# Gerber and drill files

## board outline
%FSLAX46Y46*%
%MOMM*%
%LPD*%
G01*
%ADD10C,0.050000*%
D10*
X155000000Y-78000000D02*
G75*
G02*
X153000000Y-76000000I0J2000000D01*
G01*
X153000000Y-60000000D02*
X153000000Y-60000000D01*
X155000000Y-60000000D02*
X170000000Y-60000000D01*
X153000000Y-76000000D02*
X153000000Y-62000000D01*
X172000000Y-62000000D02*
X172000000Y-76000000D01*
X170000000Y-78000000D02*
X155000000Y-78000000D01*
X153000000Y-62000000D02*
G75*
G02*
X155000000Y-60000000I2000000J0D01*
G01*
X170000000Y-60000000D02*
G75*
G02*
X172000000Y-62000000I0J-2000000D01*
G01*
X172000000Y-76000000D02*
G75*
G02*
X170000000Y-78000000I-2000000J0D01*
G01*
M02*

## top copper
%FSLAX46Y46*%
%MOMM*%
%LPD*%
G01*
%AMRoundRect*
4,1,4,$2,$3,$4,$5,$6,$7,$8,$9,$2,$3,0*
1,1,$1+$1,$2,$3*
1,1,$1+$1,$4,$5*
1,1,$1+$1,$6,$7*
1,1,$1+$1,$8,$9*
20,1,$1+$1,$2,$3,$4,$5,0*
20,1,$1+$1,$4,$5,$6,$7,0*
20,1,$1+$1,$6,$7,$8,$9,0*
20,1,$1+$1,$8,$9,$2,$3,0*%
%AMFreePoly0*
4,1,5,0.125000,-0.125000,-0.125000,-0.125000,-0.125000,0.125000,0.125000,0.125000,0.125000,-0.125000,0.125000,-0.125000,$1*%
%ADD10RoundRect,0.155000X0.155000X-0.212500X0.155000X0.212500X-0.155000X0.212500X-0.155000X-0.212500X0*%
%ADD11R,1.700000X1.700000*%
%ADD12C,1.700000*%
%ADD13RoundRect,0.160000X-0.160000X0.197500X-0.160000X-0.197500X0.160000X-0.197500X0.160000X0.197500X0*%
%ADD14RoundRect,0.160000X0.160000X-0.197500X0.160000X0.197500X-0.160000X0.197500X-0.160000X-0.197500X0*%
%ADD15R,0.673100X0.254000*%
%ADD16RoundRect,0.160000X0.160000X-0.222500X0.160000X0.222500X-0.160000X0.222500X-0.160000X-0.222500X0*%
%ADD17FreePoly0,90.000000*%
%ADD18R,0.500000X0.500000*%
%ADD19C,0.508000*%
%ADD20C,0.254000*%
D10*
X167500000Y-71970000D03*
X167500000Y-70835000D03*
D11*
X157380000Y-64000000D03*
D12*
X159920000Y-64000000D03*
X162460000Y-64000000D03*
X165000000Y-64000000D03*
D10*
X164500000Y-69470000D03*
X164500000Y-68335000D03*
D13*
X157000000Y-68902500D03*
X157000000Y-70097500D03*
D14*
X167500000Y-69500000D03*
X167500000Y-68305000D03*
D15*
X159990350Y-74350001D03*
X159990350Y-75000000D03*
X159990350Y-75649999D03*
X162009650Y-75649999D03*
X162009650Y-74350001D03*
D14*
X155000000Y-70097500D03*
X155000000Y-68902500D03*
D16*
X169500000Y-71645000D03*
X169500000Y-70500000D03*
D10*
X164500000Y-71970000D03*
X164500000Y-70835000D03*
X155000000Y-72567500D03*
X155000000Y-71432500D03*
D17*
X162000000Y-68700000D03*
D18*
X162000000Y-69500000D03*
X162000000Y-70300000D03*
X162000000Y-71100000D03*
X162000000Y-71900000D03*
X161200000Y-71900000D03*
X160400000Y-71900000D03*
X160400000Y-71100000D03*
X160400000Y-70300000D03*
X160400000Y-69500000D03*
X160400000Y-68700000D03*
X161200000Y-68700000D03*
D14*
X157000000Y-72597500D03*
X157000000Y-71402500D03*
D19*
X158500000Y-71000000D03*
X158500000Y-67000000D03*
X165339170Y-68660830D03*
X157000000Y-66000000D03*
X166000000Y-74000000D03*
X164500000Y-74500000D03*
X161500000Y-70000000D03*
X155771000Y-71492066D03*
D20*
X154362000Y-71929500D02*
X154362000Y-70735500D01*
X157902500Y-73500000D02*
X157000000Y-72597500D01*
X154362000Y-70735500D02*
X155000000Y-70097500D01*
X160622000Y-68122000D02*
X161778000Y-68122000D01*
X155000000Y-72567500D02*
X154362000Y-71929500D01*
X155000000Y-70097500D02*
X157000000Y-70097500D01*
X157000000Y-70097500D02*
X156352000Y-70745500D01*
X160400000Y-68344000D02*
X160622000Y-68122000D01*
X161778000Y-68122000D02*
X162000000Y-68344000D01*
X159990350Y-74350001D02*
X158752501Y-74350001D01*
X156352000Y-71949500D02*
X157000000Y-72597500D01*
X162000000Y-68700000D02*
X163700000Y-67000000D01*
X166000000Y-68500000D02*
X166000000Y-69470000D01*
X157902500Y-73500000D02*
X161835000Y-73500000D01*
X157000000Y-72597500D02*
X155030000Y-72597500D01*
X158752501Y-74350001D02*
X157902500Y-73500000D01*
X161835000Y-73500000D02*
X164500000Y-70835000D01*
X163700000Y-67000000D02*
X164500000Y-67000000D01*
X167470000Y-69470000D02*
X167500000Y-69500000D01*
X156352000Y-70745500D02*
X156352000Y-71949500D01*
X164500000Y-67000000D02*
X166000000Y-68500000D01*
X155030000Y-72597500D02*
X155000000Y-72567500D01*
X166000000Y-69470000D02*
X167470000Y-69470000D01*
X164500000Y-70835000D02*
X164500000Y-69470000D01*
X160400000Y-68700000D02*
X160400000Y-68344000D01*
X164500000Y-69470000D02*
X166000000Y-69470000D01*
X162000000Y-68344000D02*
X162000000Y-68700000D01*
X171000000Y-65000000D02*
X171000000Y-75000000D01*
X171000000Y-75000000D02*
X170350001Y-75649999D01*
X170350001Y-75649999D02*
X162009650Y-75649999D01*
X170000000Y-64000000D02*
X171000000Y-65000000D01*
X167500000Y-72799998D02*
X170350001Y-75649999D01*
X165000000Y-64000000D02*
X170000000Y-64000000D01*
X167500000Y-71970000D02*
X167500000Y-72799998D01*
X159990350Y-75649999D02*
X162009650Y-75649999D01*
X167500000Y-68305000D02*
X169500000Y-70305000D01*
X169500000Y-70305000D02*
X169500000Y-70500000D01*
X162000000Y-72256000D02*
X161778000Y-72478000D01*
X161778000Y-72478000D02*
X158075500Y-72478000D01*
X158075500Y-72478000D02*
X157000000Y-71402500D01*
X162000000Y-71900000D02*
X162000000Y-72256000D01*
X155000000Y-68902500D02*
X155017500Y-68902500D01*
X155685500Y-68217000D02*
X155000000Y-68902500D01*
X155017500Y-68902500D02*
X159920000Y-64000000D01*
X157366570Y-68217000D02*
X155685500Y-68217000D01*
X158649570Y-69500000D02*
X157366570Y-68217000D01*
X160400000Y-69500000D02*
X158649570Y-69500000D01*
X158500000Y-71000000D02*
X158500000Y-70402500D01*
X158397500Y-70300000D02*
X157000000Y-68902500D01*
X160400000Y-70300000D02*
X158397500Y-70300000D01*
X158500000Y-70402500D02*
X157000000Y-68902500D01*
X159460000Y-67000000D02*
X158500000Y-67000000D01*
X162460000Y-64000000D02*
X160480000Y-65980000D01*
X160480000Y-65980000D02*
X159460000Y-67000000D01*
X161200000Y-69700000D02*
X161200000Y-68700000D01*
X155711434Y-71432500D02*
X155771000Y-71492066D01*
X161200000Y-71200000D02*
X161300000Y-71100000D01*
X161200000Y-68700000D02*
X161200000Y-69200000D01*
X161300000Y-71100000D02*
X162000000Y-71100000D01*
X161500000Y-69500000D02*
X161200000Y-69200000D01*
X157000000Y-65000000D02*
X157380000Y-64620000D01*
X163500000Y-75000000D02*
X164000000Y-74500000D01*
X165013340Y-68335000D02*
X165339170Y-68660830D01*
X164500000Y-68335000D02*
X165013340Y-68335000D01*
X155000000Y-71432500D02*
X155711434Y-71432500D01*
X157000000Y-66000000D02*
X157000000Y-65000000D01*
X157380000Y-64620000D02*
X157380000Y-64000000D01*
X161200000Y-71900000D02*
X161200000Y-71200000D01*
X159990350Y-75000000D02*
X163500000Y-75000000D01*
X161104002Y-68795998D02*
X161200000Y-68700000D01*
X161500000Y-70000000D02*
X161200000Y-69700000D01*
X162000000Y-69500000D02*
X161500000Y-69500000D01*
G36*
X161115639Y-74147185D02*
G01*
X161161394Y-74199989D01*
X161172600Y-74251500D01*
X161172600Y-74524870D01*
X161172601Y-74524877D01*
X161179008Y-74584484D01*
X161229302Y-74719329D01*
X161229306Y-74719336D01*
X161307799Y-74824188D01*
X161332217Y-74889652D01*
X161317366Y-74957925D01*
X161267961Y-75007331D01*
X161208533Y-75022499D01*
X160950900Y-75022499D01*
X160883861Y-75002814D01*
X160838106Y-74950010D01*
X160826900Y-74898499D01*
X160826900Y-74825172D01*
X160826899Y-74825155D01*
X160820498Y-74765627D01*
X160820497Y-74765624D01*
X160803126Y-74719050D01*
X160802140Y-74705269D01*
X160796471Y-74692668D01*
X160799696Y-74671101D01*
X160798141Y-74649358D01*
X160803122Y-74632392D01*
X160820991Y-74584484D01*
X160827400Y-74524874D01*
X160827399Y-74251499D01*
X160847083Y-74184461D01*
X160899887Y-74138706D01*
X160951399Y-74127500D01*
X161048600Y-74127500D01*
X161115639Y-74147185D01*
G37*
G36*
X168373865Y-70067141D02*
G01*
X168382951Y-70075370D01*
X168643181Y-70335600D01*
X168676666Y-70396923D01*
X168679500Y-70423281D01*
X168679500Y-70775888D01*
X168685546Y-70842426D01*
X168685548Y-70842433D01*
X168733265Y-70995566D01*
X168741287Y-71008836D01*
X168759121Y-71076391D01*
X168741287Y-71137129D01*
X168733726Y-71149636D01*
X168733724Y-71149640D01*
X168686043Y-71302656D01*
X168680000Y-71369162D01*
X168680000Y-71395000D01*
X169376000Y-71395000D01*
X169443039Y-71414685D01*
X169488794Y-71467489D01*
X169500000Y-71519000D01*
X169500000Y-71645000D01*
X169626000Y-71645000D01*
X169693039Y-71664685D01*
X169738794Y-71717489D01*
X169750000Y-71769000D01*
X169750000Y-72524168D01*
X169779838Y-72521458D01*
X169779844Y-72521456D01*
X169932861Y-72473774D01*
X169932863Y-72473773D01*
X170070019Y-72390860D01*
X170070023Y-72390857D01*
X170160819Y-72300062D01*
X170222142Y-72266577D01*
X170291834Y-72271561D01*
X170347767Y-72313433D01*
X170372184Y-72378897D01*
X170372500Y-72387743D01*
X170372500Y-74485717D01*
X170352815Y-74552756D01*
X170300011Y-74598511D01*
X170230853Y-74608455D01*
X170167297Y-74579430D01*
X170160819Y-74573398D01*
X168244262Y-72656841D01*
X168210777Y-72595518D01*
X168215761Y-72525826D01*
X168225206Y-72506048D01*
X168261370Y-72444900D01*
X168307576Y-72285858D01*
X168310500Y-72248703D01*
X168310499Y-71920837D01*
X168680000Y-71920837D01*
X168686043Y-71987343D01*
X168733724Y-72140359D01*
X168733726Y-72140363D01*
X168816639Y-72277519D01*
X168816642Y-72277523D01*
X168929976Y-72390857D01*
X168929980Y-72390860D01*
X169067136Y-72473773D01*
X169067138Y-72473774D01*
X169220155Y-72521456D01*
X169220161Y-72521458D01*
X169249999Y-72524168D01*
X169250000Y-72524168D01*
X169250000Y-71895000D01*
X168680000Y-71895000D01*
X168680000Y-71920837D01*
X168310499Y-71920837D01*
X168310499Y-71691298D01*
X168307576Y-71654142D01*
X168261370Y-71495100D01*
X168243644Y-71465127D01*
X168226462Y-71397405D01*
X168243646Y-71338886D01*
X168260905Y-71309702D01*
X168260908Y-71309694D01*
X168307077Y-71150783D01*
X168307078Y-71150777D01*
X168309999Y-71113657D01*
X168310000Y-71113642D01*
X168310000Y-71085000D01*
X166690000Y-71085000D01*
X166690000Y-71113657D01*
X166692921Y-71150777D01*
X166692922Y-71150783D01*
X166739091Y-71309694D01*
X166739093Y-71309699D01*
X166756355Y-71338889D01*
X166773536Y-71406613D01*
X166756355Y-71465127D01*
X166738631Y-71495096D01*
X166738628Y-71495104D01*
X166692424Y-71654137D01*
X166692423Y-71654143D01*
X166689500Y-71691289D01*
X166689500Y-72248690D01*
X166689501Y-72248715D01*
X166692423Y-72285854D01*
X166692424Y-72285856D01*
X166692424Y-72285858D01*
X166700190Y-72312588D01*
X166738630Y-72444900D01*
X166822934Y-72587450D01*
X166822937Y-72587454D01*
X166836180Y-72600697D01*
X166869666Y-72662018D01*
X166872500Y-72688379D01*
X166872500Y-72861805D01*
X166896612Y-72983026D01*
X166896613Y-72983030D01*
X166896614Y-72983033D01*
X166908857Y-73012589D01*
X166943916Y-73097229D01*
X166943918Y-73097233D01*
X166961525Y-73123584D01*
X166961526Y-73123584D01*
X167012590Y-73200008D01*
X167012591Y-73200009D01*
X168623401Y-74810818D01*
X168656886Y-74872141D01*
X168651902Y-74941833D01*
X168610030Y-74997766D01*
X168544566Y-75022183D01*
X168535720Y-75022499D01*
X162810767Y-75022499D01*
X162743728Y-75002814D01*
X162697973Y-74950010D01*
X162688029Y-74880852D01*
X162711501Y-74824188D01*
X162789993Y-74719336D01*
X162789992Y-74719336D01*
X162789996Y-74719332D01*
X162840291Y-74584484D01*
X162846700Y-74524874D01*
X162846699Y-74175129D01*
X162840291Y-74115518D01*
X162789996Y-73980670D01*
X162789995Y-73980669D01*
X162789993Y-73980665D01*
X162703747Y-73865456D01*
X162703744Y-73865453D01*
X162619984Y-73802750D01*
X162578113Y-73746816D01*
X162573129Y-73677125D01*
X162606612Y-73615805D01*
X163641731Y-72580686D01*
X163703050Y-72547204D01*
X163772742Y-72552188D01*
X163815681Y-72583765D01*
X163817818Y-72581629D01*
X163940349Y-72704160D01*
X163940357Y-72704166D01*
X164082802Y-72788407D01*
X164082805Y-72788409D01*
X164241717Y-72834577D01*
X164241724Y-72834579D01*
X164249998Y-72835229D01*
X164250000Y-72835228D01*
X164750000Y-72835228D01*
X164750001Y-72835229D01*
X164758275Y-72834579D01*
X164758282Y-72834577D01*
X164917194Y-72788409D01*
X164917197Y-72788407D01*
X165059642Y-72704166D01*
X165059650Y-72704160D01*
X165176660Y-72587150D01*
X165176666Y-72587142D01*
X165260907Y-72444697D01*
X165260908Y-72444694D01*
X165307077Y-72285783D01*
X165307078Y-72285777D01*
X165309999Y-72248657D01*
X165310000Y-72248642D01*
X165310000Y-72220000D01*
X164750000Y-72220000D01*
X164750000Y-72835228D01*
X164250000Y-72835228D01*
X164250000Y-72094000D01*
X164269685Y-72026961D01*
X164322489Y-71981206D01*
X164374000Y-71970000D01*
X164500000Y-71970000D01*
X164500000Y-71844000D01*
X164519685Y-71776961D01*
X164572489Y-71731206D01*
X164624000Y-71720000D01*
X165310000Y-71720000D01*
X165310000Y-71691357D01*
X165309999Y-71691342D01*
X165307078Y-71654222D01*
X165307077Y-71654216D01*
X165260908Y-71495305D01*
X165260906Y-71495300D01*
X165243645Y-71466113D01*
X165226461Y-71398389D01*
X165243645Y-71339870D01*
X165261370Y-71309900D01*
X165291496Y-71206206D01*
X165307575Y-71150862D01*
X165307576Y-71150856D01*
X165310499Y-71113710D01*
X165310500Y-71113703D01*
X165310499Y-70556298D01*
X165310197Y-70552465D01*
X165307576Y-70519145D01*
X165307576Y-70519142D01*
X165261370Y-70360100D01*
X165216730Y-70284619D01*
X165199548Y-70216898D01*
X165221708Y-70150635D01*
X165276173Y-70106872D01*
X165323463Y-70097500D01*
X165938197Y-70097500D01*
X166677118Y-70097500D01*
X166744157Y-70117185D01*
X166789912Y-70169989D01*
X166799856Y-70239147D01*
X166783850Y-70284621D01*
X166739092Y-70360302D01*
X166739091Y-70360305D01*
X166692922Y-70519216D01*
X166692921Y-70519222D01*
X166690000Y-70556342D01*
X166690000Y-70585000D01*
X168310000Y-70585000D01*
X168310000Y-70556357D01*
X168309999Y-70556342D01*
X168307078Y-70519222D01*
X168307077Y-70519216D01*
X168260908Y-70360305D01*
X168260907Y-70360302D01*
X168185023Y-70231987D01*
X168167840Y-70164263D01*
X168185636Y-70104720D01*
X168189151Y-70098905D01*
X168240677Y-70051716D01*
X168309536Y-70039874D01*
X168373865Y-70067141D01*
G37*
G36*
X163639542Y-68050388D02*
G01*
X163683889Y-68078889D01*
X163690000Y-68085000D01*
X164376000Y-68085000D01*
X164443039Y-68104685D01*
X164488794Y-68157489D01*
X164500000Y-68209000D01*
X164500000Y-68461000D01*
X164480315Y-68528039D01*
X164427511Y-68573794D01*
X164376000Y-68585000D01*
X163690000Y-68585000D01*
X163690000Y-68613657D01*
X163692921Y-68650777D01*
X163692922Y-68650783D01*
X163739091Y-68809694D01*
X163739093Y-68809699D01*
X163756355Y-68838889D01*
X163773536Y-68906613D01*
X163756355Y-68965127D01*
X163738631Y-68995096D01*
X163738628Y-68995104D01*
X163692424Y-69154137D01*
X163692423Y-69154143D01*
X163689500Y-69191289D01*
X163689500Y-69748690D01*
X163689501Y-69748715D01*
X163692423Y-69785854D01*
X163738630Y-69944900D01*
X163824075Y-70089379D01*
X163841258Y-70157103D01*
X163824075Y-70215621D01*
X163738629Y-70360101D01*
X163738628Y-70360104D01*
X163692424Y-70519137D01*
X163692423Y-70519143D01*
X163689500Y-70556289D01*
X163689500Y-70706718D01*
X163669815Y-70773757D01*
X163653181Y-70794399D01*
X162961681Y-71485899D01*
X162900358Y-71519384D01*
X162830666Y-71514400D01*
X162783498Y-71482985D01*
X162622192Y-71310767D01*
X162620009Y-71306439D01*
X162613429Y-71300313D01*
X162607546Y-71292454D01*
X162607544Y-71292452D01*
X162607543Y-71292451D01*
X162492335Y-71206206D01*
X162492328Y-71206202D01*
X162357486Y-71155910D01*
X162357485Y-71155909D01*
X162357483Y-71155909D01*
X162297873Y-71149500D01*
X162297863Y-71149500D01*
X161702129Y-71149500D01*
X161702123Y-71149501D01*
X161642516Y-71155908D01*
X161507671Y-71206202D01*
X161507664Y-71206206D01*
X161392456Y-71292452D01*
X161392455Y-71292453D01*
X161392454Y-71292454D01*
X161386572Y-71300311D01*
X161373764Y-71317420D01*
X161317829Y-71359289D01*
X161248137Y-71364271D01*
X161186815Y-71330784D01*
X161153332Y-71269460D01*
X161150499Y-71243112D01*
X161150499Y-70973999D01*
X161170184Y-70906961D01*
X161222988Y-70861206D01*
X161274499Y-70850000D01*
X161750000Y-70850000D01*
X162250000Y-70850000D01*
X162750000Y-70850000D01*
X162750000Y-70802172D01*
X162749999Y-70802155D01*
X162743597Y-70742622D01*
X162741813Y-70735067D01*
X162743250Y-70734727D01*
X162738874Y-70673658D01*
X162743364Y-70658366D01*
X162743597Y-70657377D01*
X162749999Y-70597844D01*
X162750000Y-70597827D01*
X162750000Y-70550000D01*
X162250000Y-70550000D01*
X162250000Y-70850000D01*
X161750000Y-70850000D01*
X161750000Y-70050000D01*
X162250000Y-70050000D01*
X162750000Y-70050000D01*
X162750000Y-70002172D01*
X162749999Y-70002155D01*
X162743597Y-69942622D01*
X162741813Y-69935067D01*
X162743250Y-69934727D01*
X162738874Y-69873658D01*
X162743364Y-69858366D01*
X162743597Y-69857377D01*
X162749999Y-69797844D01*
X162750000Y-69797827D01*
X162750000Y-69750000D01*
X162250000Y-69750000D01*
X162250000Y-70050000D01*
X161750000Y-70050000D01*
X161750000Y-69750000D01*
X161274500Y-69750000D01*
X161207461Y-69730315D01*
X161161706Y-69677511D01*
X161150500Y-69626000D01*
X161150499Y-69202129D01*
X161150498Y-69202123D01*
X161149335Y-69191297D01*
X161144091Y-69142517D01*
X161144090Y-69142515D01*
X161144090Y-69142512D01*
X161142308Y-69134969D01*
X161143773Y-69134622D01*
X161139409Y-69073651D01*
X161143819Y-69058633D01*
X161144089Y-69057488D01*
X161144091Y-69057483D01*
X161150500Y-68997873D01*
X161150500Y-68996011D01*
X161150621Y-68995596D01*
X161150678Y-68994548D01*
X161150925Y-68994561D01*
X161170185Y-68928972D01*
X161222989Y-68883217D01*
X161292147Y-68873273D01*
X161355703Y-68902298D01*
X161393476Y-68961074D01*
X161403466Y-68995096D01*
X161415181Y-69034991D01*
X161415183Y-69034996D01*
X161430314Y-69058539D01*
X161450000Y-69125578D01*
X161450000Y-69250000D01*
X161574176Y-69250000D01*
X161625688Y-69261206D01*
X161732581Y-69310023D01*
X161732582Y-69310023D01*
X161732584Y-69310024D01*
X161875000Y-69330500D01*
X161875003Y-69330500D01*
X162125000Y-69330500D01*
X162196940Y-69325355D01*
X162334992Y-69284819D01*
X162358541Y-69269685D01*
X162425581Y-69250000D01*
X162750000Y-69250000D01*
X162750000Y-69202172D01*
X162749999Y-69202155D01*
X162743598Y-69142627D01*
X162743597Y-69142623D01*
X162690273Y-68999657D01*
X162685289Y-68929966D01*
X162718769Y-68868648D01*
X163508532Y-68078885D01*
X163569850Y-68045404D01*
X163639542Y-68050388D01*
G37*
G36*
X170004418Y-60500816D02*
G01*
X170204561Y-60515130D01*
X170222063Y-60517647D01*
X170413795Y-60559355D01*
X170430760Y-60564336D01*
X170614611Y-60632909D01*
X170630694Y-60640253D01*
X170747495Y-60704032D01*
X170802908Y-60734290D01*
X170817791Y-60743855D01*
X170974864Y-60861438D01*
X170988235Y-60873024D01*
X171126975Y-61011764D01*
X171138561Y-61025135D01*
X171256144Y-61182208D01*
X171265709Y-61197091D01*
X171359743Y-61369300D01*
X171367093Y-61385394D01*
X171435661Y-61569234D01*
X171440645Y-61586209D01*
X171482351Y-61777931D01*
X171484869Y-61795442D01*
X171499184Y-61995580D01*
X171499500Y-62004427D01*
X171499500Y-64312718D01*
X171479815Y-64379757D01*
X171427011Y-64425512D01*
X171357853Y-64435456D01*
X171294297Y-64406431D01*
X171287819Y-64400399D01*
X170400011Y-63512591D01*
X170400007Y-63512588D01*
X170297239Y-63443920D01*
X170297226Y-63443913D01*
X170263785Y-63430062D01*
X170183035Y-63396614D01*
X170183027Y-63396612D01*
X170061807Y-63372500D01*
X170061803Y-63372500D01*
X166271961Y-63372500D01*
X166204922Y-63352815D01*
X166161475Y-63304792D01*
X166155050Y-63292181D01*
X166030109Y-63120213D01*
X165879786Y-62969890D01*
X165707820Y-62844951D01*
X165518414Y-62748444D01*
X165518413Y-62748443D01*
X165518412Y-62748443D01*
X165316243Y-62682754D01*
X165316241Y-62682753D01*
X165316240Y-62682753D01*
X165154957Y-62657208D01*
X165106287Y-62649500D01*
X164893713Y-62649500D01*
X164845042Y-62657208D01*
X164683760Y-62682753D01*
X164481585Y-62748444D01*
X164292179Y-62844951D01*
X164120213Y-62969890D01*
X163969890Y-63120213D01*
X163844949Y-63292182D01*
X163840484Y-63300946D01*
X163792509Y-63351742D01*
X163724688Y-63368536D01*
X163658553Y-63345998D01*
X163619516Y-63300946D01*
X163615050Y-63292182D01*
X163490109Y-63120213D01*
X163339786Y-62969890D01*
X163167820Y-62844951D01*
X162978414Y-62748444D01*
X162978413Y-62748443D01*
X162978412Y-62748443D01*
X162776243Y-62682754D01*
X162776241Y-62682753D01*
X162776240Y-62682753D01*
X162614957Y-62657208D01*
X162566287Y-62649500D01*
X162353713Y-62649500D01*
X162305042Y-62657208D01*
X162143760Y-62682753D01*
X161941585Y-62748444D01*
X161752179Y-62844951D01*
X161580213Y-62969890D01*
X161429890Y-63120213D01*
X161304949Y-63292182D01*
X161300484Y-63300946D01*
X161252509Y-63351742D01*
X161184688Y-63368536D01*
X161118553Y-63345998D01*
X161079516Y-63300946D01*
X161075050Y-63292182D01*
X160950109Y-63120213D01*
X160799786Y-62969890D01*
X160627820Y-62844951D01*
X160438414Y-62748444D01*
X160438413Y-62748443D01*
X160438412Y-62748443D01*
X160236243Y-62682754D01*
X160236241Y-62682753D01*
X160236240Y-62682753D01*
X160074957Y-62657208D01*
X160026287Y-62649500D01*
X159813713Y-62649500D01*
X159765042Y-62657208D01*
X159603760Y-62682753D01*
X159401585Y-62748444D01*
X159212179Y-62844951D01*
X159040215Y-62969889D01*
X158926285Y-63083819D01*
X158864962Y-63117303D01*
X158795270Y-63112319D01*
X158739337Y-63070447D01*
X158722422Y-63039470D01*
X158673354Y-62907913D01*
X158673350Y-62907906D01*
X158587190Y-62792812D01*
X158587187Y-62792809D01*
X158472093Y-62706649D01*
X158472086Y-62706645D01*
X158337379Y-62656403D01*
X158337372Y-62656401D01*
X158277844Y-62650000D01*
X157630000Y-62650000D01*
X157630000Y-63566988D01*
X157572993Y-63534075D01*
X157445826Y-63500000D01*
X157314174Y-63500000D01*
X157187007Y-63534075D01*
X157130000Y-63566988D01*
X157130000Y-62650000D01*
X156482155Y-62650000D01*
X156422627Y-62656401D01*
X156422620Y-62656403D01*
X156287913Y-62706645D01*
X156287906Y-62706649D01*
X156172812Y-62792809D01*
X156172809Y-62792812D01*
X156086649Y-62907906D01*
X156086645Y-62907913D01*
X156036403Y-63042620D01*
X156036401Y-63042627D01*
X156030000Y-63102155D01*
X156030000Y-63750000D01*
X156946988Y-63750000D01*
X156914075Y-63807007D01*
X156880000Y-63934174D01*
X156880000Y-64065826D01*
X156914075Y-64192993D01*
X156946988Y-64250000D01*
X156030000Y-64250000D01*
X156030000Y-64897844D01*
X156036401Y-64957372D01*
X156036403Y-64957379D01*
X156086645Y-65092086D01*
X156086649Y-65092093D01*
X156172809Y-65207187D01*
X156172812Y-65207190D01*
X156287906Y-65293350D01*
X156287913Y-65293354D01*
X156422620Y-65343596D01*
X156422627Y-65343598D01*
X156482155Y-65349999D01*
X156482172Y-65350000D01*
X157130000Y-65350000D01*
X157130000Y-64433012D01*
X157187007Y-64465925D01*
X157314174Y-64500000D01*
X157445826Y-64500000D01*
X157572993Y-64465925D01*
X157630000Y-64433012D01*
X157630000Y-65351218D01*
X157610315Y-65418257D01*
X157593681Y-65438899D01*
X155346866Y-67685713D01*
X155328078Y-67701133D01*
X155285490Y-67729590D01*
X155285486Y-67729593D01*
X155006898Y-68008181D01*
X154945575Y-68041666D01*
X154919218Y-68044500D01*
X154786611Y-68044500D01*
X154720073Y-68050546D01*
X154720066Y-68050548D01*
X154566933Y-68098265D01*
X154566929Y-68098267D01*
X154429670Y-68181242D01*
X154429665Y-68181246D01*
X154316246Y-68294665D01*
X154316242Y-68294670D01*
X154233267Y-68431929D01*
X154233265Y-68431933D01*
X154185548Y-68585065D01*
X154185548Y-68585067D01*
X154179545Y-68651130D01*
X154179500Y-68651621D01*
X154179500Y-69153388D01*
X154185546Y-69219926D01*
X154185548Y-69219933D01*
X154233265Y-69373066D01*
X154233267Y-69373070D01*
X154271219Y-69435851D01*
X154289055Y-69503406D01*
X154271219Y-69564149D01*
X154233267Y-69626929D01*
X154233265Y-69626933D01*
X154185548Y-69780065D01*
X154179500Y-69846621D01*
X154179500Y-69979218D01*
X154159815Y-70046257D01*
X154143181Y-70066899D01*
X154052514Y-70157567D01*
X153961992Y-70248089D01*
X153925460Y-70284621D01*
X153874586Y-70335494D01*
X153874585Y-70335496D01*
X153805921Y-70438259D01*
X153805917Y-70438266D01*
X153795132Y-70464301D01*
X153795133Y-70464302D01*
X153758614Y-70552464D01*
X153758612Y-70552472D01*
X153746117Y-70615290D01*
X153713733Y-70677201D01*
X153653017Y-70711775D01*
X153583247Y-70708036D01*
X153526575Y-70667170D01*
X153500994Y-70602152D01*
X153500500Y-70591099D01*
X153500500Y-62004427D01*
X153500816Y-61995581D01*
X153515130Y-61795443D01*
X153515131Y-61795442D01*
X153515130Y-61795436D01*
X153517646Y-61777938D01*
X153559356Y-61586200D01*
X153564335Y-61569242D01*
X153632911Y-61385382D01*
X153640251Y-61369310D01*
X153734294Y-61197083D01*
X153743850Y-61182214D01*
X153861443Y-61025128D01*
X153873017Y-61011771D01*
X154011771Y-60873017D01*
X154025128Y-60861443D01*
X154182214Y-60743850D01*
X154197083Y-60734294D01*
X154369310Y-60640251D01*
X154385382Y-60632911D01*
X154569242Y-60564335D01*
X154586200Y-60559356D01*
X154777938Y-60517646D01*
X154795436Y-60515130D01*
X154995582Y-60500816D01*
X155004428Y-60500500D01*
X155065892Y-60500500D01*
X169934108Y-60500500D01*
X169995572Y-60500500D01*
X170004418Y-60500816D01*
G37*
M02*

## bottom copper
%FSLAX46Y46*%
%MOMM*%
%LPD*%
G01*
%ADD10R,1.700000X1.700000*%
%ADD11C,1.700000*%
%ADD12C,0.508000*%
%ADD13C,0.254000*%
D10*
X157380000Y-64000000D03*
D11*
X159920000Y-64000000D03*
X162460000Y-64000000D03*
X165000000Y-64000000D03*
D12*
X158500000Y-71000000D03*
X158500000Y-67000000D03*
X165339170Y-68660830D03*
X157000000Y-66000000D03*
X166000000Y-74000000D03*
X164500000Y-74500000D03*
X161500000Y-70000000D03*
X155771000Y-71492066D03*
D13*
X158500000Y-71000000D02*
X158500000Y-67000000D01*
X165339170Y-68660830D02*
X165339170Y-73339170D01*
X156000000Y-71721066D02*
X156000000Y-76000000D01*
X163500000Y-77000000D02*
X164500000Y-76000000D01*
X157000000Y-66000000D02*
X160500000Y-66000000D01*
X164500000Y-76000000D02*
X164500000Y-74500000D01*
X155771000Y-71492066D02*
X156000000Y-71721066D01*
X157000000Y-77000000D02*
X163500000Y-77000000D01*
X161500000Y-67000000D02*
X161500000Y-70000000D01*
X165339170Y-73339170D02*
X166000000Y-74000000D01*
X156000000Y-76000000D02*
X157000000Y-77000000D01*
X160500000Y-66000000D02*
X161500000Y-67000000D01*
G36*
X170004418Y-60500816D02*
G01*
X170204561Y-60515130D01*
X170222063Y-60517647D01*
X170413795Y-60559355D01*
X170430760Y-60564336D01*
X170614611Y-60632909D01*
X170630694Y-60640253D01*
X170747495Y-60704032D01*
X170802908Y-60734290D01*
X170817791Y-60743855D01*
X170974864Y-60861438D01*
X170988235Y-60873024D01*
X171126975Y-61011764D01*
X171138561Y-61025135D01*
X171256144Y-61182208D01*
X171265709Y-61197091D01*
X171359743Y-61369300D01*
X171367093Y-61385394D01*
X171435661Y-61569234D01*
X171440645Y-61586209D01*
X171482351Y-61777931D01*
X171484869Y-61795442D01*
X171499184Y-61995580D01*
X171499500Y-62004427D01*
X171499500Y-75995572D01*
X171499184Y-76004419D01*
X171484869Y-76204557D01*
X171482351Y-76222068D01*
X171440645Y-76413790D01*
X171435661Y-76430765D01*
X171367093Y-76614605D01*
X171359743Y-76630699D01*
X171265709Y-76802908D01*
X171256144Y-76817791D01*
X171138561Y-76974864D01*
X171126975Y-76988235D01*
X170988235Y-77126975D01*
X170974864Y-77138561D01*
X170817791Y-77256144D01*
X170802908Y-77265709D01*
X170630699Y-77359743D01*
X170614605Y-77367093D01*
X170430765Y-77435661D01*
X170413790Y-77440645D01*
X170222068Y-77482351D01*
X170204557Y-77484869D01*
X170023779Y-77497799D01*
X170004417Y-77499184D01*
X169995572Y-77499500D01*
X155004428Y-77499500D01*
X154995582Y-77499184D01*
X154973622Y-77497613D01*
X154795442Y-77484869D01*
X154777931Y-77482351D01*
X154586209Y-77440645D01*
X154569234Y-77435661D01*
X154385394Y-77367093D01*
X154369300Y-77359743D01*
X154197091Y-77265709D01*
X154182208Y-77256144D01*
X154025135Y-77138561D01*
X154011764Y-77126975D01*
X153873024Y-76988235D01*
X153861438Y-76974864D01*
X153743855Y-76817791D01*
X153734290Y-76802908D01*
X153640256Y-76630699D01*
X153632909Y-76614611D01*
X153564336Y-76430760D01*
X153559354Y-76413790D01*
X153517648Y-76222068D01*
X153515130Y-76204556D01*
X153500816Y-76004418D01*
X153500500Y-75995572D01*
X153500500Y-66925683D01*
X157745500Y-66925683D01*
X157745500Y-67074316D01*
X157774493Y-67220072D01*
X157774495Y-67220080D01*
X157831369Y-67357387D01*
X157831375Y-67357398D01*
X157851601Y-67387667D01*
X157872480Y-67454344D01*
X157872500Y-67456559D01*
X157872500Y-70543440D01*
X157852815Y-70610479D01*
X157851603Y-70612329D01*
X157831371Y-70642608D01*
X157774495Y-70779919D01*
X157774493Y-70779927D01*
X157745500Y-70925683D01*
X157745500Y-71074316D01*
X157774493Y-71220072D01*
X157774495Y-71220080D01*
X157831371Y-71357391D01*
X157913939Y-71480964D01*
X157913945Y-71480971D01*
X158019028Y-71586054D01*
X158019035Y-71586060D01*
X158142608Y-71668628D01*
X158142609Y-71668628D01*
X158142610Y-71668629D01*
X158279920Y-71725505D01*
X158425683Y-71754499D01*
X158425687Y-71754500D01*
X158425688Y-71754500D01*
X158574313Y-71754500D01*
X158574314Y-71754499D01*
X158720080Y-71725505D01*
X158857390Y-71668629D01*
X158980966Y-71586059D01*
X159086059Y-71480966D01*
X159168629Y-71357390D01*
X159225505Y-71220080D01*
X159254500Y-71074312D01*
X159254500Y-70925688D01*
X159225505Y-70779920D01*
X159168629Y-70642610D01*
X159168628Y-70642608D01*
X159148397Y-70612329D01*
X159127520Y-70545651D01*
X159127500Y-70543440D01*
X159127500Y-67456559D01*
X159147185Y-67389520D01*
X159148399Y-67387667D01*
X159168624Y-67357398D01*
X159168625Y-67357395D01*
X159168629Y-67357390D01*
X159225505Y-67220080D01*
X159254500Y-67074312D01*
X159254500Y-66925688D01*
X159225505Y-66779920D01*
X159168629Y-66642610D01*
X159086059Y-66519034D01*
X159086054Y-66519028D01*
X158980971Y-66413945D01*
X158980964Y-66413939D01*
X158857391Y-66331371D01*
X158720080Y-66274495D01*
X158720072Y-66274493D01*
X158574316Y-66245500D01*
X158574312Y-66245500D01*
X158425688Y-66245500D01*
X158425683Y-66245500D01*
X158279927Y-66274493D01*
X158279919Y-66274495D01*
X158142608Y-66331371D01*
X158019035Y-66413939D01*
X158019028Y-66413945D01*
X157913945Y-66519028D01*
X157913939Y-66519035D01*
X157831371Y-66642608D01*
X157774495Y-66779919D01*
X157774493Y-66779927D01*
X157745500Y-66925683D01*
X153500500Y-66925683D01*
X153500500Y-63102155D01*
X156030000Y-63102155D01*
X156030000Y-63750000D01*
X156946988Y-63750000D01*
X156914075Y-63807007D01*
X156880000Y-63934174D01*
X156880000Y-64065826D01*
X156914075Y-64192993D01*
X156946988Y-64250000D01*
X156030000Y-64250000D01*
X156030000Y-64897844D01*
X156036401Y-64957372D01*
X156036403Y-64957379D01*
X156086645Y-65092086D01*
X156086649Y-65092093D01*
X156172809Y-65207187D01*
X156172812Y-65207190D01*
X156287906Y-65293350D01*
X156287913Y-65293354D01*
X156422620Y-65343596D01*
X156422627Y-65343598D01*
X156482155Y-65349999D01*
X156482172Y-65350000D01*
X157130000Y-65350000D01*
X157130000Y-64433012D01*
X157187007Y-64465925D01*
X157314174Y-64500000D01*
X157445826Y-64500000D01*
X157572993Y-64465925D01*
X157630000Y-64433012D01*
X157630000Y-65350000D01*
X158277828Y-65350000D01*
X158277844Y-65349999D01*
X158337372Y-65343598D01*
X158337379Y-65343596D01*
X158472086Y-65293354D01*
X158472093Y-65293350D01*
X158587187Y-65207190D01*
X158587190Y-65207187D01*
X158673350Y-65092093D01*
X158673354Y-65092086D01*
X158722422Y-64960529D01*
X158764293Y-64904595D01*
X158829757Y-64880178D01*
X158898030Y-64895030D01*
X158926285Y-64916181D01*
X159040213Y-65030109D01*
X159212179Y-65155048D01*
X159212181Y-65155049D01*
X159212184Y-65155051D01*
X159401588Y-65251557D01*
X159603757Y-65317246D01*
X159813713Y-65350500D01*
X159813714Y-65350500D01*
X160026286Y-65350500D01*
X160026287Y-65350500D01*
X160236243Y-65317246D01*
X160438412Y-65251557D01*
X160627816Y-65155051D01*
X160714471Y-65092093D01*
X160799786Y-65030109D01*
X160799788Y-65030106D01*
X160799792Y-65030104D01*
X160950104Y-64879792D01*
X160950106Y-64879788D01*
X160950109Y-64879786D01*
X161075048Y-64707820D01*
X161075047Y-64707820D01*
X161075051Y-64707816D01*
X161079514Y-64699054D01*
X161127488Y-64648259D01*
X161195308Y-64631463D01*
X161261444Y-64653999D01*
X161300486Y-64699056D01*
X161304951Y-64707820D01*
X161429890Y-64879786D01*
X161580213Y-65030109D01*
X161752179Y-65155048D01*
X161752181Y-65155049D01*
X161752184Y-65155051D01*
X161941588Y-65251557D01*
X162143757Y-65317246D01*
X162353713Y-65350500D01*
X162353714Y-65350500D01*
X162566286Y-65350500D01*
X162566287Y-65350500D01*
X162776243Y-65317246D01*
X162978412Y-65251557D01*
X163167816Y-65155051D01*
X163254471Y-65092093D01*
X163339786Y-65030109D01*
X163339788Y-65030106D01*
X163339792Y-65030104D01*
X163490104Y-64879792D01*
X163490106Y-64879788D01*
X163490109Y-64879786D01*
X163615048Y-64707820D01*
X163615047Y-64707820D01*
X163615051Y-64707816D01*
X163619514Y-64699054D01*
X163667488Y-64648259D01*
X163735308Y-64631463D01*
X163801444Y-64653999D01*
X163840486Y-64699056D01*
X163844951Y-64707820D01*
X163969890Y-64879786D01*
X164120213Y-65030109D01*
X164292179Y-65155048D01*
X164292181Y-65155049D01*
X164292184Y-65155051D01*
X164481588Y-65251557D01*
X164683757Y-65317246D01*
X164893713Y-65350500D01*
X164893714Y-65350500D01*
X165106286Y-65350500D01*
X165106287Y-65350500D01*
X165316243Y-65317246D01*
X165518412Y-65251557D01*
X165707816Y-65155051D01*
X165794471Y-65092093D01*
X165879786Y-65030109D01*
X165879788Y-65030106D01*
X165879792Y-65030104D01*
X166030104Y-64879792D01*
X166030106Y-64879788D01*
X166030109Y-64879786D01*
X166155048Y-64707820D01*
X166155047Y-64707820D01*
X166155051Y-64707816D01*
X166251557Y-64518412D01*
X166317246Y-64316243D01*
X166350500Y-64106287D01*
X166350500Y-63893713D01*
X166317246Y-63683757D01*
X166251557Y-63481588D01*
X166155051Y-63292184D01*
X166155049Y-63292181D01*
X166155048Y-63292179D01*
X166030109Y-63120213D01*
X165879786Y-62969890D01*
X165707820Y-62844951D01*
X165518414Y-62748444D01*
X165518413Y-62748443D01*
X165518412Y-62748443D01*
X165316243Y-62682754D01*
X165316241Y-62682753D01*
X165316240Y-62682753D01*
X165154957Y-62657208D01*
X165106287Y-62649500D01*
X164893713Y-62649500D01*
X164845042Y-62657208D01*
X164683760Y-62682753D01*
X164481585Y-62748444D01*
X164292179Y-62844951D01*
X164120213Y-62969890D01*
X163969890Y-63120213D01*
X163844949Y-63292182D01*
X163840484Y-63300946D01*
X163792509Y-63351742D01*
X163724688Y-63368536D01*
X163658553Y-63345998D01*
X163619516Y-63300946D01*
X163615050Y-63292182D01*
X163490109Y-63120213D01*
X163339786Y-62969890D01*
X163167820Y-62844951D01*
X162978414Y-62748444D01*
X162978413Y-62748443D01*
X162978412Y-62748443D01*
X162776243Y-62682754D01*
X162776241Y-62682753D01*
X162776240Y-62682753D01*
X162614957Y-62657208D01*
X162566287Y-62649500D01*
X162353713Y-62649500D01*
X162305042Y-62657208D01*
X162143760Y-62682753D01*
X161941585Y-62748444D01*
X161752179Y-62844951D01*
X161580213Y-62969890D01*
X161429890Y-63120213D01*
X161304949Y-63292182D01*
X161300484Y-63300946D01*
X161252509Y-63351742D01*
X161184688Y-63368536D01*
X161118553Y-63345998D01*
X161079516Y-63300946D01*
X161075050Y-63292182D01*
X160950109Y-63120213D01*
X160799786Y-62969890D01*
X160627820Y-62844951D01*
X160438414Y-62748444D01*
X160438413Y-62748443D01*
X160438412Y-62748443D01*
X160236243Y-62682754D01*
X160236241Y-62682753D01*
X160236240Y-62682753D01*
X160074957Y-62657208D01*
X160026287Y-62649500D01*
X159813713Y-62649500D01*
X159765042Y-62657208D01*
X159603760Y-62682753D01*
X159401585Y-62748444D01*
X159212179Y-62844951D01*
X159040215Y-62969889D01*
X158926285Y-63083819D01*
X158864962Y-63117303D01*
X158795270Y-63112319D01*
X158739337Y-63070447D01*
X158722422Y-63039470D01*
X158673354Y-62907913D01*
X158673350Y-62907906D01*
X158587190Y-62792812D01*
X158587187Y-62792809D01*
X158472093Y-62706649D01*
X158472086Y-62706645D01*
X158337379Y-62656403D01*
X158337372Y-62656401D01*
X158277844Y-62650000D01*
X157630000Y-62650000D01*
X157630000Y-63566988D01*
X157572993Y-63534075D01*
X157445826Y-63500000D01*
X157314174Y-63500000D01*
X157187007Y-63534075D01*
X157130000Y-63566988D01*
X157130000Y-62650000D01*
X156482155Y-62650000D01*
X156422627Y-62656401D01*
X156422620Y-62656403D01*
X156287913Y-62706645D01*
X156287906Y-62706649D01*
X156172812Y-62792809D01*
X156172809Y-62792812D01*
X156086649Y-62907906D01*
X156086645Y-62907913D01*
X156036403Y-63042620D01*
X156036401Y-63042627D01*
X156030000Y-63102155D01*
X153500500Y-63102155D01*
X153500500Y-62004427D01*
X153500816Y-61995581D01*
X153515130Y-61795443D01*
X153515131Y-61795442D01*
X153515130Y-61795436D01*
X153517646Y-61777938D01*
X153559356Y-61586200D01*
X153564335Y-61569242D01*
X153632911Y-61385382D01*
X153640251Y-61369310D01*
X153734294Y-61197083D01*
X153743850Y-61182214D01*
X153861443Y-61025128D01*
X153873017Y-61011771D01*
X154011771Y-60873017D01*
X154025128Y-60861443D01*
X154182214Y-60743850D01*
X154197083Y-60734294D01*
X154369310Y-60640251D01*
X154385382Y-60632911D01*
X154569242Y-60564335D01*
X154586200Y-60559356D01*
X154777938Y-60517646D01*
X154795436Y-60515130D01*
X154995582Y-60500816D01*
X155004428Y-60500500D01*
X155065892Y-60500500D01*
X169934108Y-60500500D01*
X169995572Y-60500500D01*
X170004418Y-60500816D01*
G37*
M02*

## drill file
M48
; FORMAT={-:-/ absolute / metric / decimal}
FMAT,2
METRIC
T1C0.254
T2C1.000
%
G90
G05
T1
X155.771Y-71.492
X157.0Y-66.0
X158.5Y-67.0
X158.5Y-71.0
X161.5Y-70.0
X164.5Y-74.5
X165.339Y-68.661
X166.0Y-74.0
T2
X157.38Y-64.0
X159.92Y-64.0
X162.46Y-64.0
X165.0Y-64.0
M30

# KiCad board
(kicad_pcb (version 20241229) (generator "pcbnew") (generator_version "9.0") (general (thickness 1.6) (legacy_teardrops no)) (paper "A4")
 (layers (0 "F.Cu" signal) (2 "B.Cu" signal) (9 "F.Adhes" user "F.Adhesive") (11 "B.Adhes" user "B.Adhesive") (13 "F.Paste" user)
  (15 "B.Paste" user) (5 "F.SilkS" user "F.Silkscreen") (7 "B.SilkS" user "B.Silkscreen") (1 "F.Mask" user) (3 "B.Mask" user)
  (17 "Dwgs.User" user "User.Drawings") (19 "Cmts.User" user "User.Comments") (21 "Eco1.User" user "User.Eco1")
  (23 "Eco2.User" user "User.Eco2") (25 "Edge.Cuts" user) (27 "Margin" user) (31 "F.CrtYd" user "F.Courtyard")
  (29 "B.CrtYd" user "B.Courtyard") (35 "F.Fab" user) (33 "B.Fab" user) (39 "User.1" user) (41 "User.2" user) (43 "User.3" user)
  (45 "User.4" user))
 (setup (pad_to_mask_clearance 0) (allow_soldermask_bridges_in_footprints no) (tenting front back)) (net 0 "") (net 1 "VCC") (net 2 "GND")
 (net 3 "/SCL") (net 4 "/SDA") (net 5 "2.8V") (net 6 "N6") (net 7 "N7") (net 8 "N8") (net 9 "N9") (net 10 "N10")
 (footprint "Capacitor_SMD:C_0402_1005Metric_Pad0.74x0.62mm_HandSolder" (layer "F.Cu") (at 167.5 71.4025 90)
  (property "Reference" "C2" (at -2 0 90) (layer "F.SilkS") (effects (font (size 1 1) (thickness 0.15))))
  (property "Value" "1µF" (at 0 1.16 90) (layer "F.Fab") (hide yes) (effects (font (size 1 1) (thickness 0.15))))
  (pad "1" smd roundrect (at -0.5675 0 90) (size 0.735 0.62) (layers "F.Cu" "F.Mask" "F.Paste") (roundrect_rratio 0.25) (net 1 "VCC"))
  (pad "2" smd roundrect (at 0.5675 0 90) (size 0.735 0.62) (layers "F.Cu" "F.Mask" "F.Paste") (roundrect_rratio 0.25) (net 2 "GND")))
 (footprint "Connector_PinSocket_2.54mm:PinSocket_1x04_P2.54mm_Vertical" (layer "F.Cu") (at 157.38 64 90)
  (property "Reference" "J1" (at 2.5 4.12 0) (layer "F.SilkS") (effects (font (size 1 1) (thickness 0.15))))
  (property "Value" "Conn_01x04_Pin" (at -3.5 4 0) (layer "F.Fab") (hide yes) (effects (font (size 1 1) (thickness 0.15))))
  (pad "1" thru_hole rect (at 0 0 90) (size 1.7 1.7) (drill 1) (layers "*.Cu" "*.Mask") (remove_unused_layers no) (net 2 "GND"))
  (pad "2" thru_hole circle (at 0 2.54 90) (size 1.7 1.7) (drill 1) (layers "*.Cu" "*.Mask") (remove_unused_layers no) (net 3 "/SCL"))
  (pad "3" thru_hole circle (at 0 5.08 90) (size 1.7 1.7) (drill 1) (layers "*.Cu" "*.Mask") (remove_unused_layers no) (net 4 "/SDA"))
  (pad "4" thru_hole circle (at 0 7.62 90) (size 1.7 1.7) (drill 1) (layers "*.Cu" "*.Mask") (remove_unused_layers no) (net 1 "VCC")))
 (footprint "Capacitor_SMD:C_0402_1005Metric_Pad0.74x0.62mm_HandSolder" (layer "F.Cu") (at 164.5 68.9025 90)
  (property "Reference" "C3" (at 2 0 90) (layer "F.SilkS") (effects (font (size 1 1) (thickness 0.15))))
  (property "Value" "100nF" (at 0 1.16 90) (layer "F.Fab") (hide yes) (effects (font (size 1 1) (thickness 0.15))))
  (pad "1" smd roundrect (at -0.5675 0 90) (size 0.735 0.62) (layers "F.Cu" "F.Mask" "F.Paste") (roundrect_rratio 0.25) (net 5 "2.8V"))
  (pad "2" smd roundrect (at 0.5675 0 90) (size 0.735 0.62) (layers "F.Cu" "F.Mask" "F.Paste") (roundrect_rratio 0.25) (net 2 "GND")))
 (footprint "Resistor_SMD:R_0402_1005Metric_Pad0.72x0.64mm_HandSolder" (layer "F.Cu") (at 157 69.5 -90)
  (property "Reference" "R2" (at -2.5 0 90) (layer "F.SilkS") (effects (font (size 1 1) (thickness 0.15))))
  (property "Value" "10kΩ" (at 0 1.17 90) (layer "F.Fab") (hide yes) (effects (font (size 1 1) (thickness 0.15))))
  (pad "1" smd roundrect (at -0.5975 0 270) (size 0.715 0.64) (layers "F.Cu" "F.Mask" "F.Paste") (roundrect_rratio 0.25) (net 4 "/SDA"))
  (pad "2" smd roundrect (at 0.5975 0 270) (size 0.715 0.64) (layers "F.Cu" "F.Mask" "F.Paste") (roundrect_rratio 0.25) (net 5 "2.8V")))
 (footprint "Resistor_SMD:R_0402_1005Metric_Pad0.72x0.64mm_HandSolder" (layer "F.Cu") (at 167.5 68.9025 90)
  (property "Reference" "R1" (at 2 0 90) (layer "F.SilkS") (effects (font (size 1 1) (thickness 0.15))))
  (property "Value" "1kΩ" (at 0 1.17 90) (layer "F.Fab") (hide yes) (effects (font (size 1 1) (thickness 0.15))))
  (pad "1" smd roundrect (at -0.5975 0 90) (size 0.715 0.64) (layers "F.Cu" "F.Mask" "F.Paste") (roundrect_rratio 0.25) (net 5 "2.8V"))
  (pad "2" smd roundrect (at 0.5975 0 90) (size 0.715 0.64) (layers "F.Cu" "F.Mask" "F.Paste") (roundrect_rratio 0.25) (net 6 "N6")))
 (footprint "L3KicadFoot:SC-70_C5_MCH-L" (layer "F.Cu") (at 161 75)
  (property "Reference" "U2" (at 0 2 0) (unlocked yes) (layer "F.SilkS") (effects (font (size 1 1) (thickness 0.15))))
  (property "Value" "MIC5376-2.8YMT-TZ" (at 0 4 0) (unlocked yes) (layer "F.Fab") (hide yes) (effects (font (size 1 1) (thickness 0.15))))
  (pad "1" smd rect (at -1.00965 -0.649999) (size 0.6731 0.254) (layers "F.Cu" "F.Mask" "F.Paste") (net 5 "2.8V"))
  (pad "2" smd rect (at -1.00965 0) (size 0.6731 0.254) (layers "F.Cu" "F.Mask" "F.Paste") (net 2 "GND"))
  (pad "3" smd rect (at -1.00965 0.649999) (size 0.6731 0.254) (layers "F.Cu" "F.Mask" "F.Paste") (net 1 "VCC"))
  (pad "4" smd rect (at 1.00965 0.649999) (size 0.6731 0.254) (layers "F.Cu" "F.Mask" "F.Paste") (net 1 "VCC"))
  (pad "5" smd rect (at 1.00965 -0.649999) (size 0.6731 0.254) (layers "F.Cu" "F.Mask" "F.Paste") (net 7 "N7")))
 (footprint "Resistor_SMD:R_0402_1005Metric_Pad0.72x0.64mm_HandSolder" (layer "F.Cu") (at 155 69.5 90)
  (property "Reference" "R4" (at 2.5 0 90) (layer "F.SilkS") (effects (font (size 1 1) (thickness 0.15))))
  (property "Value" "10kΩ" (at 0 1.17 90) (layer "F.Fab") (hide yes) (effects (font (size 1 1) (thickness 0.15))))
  (pad "1" smd roundrect (at -0.5975 0 90) (size 0.715 0.64) (layers "F.Cu" "F.Mask" "F.Paste") (roundrect_rratio 0.25) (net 5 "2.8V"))
  (pad "2" smd roundrect (at 0.5975 0 90) (size 0.715 0.64) (layers "F.Cu" "F.Mask" "F.Paste") (roundrect_rratio 0.25) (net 3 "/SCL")))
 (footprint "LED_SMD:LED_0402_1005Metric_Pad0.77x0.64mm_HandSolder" (layer "F.Cu") (at 169.5 71.0725 90)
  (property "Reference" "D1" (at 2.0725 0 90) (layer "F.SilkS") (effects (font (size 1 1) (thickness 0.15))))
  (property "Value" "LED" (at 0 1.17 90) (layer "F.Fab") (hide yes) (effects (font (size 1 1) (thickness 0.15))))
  (pad "1" smd roundrect (at -0.5725 0 90) (size 0.765 0.64) (layers "F.Cu" "F.Mask" "F.Paste") (roundrect_rratio 0.25) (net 2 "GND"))
  (pad "2" smd roundrect (at 0.5725 0 90) (size 0.765 0.64) (layers "F.Cu" "F.Mask" "F.Paste") (roundrect_rratio 0.25) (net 6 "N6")))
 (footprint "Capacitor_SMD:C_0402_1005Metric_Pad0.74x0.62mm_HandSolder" (layer "F.Cu") (at 164.5 71.4025 90)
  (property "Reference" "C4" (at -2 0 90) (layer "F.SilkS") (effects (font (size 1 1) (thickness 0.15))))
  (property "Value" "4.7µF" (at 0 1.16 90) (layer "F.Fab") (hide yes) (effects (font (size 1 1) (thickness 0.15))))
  (pad "1" smd roundrect (at -0.5675 0 90) (size 0.735 0.62) (layers "F.Cu" "F.Mask" "F.Paste") (roundrect_rratio 0.25) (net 2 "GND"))
  (pad "2" smd roundrect (at 0.5675 0 90) (size 0.735 0.62) (layers "F.Cu" "F.Mask" "F.Paste") (roundrect_rratio 0.25) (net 5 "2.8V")))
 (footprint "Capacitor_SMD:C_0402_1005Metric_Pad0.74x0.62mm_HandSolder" (layer "F.Cu") (at 155 72 90)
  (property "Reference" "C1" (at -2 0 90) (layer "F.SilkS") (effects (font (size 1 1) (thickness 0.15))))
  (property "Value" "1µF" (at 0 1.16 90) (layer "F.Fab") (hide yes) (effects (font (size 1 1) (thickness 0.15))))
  (pad "1" smd roundrect (at -0.5675 0 90) (size 0.735 0.62) (layers "F.Cu" "F.Mask" "F.Paste") (roundrect_rratio 0.25) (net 5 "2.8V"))
  (pad "2" smd roundrect (at 0.5675 0 90) (size 0.735 0.62) (layers "F.Cu" "F.Mask" "F.Paste") (roundrect_rratio 0.25) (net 2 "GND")))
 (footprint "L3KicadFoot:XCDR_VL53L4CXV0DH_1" (layer "F.Cu") (at 161.2 70.3 90)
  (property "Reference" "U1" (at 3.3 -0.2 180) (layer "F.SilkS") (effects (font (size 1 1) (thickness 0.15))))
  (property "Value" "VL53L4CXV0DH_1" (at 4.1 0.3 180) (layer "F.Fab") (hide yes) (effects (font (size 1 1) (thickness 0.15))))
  (pad "1" smd custom (at 1.6 0.8 90) (size 0.25 0.25) (layers "F.Cu") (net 5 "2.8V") (options (clearance outline) (anchor rect))
   (primitives))
  (pad "2" smd rect (at 0.8 0.8 90) (size 0.5 0.5) (layers "F.Cu" "F.Mask" "F.Paste") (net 2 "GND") (solder_mask_margin 0.102))
  (pad "3" smd rect (at 0 0.8 90) (size 0.5 0.5) (layers "F.Cu" "F.Mask" "F.Paste") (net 2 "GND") (solder_mask_margin 0.102))
  (pad "4" smd rect (at -0.8 0.8 90) (size 0.5 0.5) (layers "F.Cu" "F.Mask" "F.Paste") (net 2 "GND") (solder_mask_margin 0.102))
  (pad "5" smd rect (at -1.6 0.8 90) (size 0.5 0.5) (layers "F.Cu" "F.Mask" "F.Paste") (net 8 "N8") (solder_mask_margin 0.102))
  (pad "6" smd rect (at -1.6 0 90) (size 0.5 0.5) (layers "F.Cu" "F.Mask" "F.Paste") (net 2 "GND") (solder_mask_margin 0.102))
  (pad "7" smd rect (at -1.6 -0.8 90) (size 0.5 0.5) (layers "F.Cu" "F.Mask" "F.Paste") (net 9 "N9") (solder_mask_margin 0.102))
  (pad "8" smd rect (at -0.8 -0.8 90) (size 0.5 0.5) (layers "F.Cu" "F.Mask" "F.Paste") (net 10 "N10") (solder_mask_margin 0.102))
  (pad "9" smd rect (at 0 -0.8 90) (size 0.5 0.5) (layers "F.Cu" "F.Mask" "F.Paste") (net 4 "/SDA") (solder_mask_margin 0.102))
  (pad "10" smd rect (at 0.8 -0.8 90) (size 0.5 0.5) (layers "F.Cu" "F.Mask" "F.Paste") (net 3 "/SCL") (solder_mask_margin 0.102))
  (pad "11" smd rect (at 1.6 -0.8 90) (size 0.5 0.5) (layers "F.Cu" "F.Mask" "F.Paste") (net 5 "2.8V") (solder_mask_margin 0.102))
  (pad "12" smd rect (at 1.6 0 90) (size 0.5 0.5) (layers "F.Cu" "F.Mask" "F.Paste") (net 2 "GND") (solder_mask_margin 0.102)))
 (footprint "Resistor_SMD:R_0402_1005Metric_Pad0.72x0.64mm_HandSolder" (layer "F.Cu") (at 157 72 90)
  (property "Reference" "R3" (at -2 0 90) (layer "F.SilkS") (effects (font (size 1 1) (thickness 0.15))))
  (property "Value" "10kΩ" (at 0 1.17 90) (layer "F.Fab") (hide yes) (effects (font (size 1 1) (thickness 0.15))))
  (pad "1" smd roundrect (at -0.5975 0 90) (size 0.715 0.64) (layers "F.Cu" "F.Mask" "F.Paste") (roundrect_rratio 0.25) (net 5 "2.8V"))
  (pad "2" smd roundrect (at 0.5975 0 90) (size 0.715 0.64) (layers "F.Cu" "F.Mask" "F.Paste") (roundrect_rratio 0.25) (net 8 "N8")))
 (gr_arc (start 155 78) (mid 153.585786 77.414214) (end 153 76) (stroke (width 0.05) (type default)) (layer "Edge.Cuts"))
 (gr_line (start 153 60) (end 153 60) (stroke (width 0.05) (type default)) (layer "Edge.Cuts"))
 (gr_line (start 155 60) (end 170 60) (stroke (width 0.05) (type default)) (layer "Edge.Cuts"))
 (gr_line (start 153 76) (end 153 62) (stroke (width 0.05) (type default)) (layer "Edge.Cuts"))
 (gr_line (start 172 62) (end 172 76) (stroke (width 0.05) (type default)) (layer "Edge.Cuts"))
 (gr_line (start 170 78) (end 155 78) (stroke (width 0.05) (type default)) (layer "Edge.Cuts"))
 (gr_arc (start 153 62) (mid 153.585786 60.585786) (end 155 60) (stroke (width 0.05) (type default)) (layer "Edge.Cuts"))
 (gr_arc (start 170 60) (mid 171.414214 60.585786) (end 172 62) (stroke (width 0.05) (type default)) (layer "Edge.Cuts"))
 (gr_arc (start 172 76) (mid 171.414214 77.414214) (end 170 78) (stroke (width 0.05) (type default)) (layer "Edge.Cuts"))
 (segment (start 154.362 71.9295) (end 154.362 70.7355) (width 0.254) (layer "F.Cu") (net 5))
 (segment (start 157.9025 73.5) (end 157 72.5975) (width 0.254) (layer "F.Cu") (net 5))
 (segment (start 154.362 70.7355) (end 155 70.0975) (width 0.254) (layer "F.Cu") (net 5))
 (segment (start 160.622 68.122) (end 161.778 68.122) (width 0.254) (layer "F.Cu") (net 5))
 (segment (start 155 72.5675) (end 154.362 71.9295) (width 0.254) (layer "F.Cu") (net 5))
 (segment (start 155 70.0975) (end 157 70.0975) (width 0.254) (layer "F.Cu") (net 5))
 (segment (start 157 70.0975) (end 156.352 70.7455) (width 0.254) (layer "F.Cu") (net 5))
 (segment (start 160.4 68.344) (end 160.622 68.122) (width 0.254) (layer "F.Cu") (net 5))
 (segment (start 161.778 68.122) (end 162 68.344) (width 0.254) (layer "F.Cu") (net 5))
 (segment (start 159.99035 74.350001) (end 158.752501 74.350001) (width 0.254) (layer "F.Cu") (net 5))
 (segment (start 156.352 71.9495) (end 157 72.5975) (width 0.254) (layer "F.Cu") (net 5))
 (segment (start 162 68.7) (end 163.7 67) (width 0.254) (layer "F.Cu") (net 5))
 (segment (start 166 68.5) (end 166 69.47) (width 0.254) (layer "F.Cu") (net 5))
 (segment (start 157.9025 73.5) (end 161.835 73.5) (width 0.254) (layer "F.Cu") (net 5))
 (segment (start 157 72.5975) (end 155.03 72.5975) (width 0.254) (layer "F.Cu") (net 5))
 (segment (start 158.752501 74.350001) (end 157.9025 73.5) (width 0.254) (layer "F.Cu") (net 5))
 (segment (start 161.835 73.5) (end 164.5 70.835) (width 0.254) (layer "F.Cu") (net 5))
 (segment (start 163.7 67) (end 164.5 67) (width 0.254) (layer "F.Cu") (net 5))
 (segment (start 167.47 69.47) (end 167.5 69.5) (width 0.254) (layer "F.Cu") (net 5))
 (segment (start 156.352 70.7455) (end 156.352 71.9495) (width 0.254) (layer "F.Cu") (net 5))
 (segment (start 164.5 67) (end 166 68.5) (width 0.254) (layer "F.Cu") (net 5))
 (segment (start 155.03 72.5975) (end 155 72.5675) (width 0.254) (layer "F.Cu") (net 5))
 (segment (start 166 69.47) (end 167.47 69.47) (width 0.254) (layer "F.Cu") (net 5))
 (segment (start 164.5 70.835) (end 164.5 69.47) (width 0.254) (layer "F.Cu") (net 5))
 (segment (start 160.4 68.7) (end 160.4 68.344) (width 0.254) (layer "F.Cu") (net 5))
 (segment (start 164.5 69.47) (end 166 69.47) (width 0.254) (layer "F.Cu") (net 5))
 (segment (start 162 68.344) (end 162 68.7) (width 0.254) (layer "F.Cu") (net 5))
 (segment (start 171 65) (end 171 75) (width 0.254) (layer "F.Cu") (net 1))
 (segment (start 171 75) (end 170.350001 75.649999) (width 0.254) (layer "F.Cu") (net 1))
 (segment (start 170.350001 75.649999) (end 162.00965 75.649999) (width 0.254) (layer "F.Cu") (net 1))
 (segment (start 170 64) (end 171 65) (width 0.254) (layer "F.Cu") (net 1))
 (segment (start 167.5 72.799998) (end 170.350001 75.649999) (width 0.254) (layer "F.Cu") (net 1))
 (segment (start 165 64) (end 170 64) (width 0.254) (layer "F.Cu") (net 1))
 (segment (start 167.5 71.97) (end 167.5 72.799998) (width 0.254) (layer "F.Cu") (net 1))
 (segment (start 159.99035 75.649999) (end 162.00965 75.649999) (width 0.254) (layer "F.Cu") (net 1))
 (segment (start 167.5 68.305) (end 169.5 70.305) (width 0.254) (layer "F.Cu") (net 6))
 (segment (start 169.5 70.305) (end 169.5 70.5) (width 0.254) (layer "F.Cu") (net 6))
 (segment (start 162 72.256) (end 161.778 72.478) (width 0.254) (layer "F.Cu") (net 8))
 (segment (start 161.778 72.478) (end 158.0755 72.478) (width 0.254) (layer "F.Cu") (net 8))
 (segment (start 158.0755 72.478) (end 157 71.4025) (width 0.254) (layer "F.Cu") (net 8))
 (segment (start 162 71.9) (end 162 72.256) (width 0.254) (layer "F.Cu") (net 8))
 (segment (start 155 68.9025) (end 155.0175 68.9025) (width 0.254) (layer "F.Cu") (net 3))
 (segment (start 155.6855 68.217) (end 155 68.9025) (width 0.254) (layer "F.Cu") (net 3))
 (segment (start 155.0175 68.9025) (end 159.92 64) (width 0.254) (layer "F.Cu") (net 3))
 (segment (start 157.36657 68.217) (end 155.6855 68.217) (width 0.254) (layer "F.Cu") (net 3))
 (segment (start 158.64957 69.5) (end 157.36657 68.217) (width 0.254) (layer "F.Cu") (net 3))
 (segment (start 160.4 69.5) (end 158.64957 69.5) (width 0.254) (layer "F.Cu") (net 3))
 (segment (start 158.5 71) (end 158.5 70.4025) (width 0.254) (layer "F.Cu") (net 4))
 (segment (start 158.3975 70.3) (end 157 68.9025) (width 0.254) (layer "F.Cu") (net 4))
 (segment (start 160.4 70.3) (end 158.3975 70.3) (width 0.254) (layer "F.Cu") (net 4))
 (segment (start 158.5 70.4025) (end 157 68.9025) (width 0.254) (layer "F.Cu") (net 4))
 (segment (start 159.46 67) (end 158.5 67) (width 0.254) (layer "F.Cu") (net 4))
 (segment (start 162.46 64) (end 160.48 65.98) (width 0.254) (layer "F.Cu") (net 4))
 (segment (start 160.48 65.98) (end 159.46 67) (width 0.254) (layer "F.Cu") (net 4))
 (via (at 158.5 71) (size 0.508) (drill 0.254) (layers "F.Cu" "B.Cu") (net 4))
 (via (at 158.5 67) (size 0.508) (drill 0.254) (layers "F.Cu" "B.Cu") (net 4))
 (segment (start 158.5 71) (end 158.5 67) (width 0.254) (layer "B.Cu") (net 4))
 (segment (start 161.2 69.7) (end 161.2 68.7) (width 0.254) (layer "F.Cu") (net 2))
 (segment (start 155.711434 71.4325) (end 155.771 71.492066) (width 0.254) (layer "F.Cu") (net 2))
 (segment (start 161.2 71.2) (end 161.3 71.1) (width 0.254) (layer "F.Cu") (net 2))
 (segment (start 161.2 68.7) (end 161.2 69.2) (width 0.254) (layer "F.Cu") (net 2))
 (segment (start 161.3 71.1) (end 162 71.1) (width 0.254) (layer "F.Cu") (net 2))
 (segment (start 161.5 69.5) (end 161.2 69.2) (width 0.254) (layer "F.Cu") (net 2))
 (segment (start 157 65) (end 157.38 64.62) (width 0.254) (layer "F.Cu") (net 2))
 (segment (start 163.5 75) (end 164 74.5) (width 0.254) (layer "F.Cu") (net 2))
 (segment (start 165.01334 68.335) (end 165.33917 68.66083) (width 0.254) (layer "F.Cu") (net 2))
 (segment (start 164.5 68.335) (end 165.01334 68.335) (width 0.254) (layer "F.Cu") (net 2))
 (segment (start 155 71.4325) (end 155.711434 71.4325) (width 0.254) (layer "F.Cu") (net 2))
 (segment (start 157 66) (end 157 65) (width 0.254) (layer "F.Cu") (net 2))
 (segment (start 157.38 64.62) (end 157.38 64) (width 0.254) (layer "F.Cu") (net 2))
 (segment (start 161.2 71.9) (end 161.2 71.2) (width 0.254) (layer "F.Cu") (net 2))
 (segment (start 159.99035 75) (end 163.5 75) (width 0.254) (layer "F.Cu") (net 2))
 (segment (start 161.104002 68.795998) (end 161.2 68.7) (width 0.254) (layer "F.Cu") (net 2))
 (segment (start 161.5 70) (end 161.2 69.7) (width 0.254) (layer "F.Cu") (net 2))
 (segment (start 162 69.5) (end 161.5 69.5) (width 0.254) (layer "F.Cu") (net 2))
 (via (at 165.33917 68.66083) (size 0.508) (drill 0.254) (layers "F.Cu" "B.Cu") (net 2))
 (via (at 157 66) (size 0.508) (drill 0.254) (layers "F.Cu" "B.Cu") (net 2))
 (via (at 166 74) (size 0.508) (drill 0.254) (layers "F.Cu" "B.Cu") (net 2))
 (via (at 164.5 74.5) (size 0.508) (drill 0.254) (layers "F.Cu" "B.Cu") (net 2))
 (via (at 161.5 70) (size 0.508) (drill 0.254) (layers "F.Cu" "B.Cu") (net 2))
 (via (at 155.771 71.492066) (size 0.508) (drill 0.254) (layers "F.Cu" "B.Cu") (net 2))
 (segment (start 165.33917 68.66083) (end 165.33917 73.33917) (width 0.254) (layer "B.Cu") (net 2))
 (segment (start 156 71.721066) (end 156 76) (width 0.254) (layer "B.Cu") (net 2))
 (segment (start 163.5 77) (end 164.5 76) (width 0.254) (layer "B.Cu") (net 2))
 (segment (start 157 66) (end 160.5 66) (width 0.254) (layer "B.Cu") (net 2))
 (segment (start 164.5 76) (end 164.5 74.5) (width 0.254) (layer "B.Cu") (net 2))
 (segment (start 155.771 71.492066) (end 156 71.721066) (width 0.254) (layer "B.Cu") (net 2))
 (segment (start 157 77) (end 163.5 77) (width 0.254) (layer "B.Cu") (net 2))
 (segment (start 161.5 67) (end 161.5 70) (width 0.254) (layer "B.Cu") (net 2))
 (segment (start 165.33917 73.33917) (end 166 74) (width 0.254) (layer "B.Cu") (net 2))
 (segment (start 156 76) (end 157 77) (width 0.254) (layer "B.Cu") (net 2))
 (segment (start 160.5 66) (end 161.5 67) (width 0.254) (layer "B.Cu") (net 2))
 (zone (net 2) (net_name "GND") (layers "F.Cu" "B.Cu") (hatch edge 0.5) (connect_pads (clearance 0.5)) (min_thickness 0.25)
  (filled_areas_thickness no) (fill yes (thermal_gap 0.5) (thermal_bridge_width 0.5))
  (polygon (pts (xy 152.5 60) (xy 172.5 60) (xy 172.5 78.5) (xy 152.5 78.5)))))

